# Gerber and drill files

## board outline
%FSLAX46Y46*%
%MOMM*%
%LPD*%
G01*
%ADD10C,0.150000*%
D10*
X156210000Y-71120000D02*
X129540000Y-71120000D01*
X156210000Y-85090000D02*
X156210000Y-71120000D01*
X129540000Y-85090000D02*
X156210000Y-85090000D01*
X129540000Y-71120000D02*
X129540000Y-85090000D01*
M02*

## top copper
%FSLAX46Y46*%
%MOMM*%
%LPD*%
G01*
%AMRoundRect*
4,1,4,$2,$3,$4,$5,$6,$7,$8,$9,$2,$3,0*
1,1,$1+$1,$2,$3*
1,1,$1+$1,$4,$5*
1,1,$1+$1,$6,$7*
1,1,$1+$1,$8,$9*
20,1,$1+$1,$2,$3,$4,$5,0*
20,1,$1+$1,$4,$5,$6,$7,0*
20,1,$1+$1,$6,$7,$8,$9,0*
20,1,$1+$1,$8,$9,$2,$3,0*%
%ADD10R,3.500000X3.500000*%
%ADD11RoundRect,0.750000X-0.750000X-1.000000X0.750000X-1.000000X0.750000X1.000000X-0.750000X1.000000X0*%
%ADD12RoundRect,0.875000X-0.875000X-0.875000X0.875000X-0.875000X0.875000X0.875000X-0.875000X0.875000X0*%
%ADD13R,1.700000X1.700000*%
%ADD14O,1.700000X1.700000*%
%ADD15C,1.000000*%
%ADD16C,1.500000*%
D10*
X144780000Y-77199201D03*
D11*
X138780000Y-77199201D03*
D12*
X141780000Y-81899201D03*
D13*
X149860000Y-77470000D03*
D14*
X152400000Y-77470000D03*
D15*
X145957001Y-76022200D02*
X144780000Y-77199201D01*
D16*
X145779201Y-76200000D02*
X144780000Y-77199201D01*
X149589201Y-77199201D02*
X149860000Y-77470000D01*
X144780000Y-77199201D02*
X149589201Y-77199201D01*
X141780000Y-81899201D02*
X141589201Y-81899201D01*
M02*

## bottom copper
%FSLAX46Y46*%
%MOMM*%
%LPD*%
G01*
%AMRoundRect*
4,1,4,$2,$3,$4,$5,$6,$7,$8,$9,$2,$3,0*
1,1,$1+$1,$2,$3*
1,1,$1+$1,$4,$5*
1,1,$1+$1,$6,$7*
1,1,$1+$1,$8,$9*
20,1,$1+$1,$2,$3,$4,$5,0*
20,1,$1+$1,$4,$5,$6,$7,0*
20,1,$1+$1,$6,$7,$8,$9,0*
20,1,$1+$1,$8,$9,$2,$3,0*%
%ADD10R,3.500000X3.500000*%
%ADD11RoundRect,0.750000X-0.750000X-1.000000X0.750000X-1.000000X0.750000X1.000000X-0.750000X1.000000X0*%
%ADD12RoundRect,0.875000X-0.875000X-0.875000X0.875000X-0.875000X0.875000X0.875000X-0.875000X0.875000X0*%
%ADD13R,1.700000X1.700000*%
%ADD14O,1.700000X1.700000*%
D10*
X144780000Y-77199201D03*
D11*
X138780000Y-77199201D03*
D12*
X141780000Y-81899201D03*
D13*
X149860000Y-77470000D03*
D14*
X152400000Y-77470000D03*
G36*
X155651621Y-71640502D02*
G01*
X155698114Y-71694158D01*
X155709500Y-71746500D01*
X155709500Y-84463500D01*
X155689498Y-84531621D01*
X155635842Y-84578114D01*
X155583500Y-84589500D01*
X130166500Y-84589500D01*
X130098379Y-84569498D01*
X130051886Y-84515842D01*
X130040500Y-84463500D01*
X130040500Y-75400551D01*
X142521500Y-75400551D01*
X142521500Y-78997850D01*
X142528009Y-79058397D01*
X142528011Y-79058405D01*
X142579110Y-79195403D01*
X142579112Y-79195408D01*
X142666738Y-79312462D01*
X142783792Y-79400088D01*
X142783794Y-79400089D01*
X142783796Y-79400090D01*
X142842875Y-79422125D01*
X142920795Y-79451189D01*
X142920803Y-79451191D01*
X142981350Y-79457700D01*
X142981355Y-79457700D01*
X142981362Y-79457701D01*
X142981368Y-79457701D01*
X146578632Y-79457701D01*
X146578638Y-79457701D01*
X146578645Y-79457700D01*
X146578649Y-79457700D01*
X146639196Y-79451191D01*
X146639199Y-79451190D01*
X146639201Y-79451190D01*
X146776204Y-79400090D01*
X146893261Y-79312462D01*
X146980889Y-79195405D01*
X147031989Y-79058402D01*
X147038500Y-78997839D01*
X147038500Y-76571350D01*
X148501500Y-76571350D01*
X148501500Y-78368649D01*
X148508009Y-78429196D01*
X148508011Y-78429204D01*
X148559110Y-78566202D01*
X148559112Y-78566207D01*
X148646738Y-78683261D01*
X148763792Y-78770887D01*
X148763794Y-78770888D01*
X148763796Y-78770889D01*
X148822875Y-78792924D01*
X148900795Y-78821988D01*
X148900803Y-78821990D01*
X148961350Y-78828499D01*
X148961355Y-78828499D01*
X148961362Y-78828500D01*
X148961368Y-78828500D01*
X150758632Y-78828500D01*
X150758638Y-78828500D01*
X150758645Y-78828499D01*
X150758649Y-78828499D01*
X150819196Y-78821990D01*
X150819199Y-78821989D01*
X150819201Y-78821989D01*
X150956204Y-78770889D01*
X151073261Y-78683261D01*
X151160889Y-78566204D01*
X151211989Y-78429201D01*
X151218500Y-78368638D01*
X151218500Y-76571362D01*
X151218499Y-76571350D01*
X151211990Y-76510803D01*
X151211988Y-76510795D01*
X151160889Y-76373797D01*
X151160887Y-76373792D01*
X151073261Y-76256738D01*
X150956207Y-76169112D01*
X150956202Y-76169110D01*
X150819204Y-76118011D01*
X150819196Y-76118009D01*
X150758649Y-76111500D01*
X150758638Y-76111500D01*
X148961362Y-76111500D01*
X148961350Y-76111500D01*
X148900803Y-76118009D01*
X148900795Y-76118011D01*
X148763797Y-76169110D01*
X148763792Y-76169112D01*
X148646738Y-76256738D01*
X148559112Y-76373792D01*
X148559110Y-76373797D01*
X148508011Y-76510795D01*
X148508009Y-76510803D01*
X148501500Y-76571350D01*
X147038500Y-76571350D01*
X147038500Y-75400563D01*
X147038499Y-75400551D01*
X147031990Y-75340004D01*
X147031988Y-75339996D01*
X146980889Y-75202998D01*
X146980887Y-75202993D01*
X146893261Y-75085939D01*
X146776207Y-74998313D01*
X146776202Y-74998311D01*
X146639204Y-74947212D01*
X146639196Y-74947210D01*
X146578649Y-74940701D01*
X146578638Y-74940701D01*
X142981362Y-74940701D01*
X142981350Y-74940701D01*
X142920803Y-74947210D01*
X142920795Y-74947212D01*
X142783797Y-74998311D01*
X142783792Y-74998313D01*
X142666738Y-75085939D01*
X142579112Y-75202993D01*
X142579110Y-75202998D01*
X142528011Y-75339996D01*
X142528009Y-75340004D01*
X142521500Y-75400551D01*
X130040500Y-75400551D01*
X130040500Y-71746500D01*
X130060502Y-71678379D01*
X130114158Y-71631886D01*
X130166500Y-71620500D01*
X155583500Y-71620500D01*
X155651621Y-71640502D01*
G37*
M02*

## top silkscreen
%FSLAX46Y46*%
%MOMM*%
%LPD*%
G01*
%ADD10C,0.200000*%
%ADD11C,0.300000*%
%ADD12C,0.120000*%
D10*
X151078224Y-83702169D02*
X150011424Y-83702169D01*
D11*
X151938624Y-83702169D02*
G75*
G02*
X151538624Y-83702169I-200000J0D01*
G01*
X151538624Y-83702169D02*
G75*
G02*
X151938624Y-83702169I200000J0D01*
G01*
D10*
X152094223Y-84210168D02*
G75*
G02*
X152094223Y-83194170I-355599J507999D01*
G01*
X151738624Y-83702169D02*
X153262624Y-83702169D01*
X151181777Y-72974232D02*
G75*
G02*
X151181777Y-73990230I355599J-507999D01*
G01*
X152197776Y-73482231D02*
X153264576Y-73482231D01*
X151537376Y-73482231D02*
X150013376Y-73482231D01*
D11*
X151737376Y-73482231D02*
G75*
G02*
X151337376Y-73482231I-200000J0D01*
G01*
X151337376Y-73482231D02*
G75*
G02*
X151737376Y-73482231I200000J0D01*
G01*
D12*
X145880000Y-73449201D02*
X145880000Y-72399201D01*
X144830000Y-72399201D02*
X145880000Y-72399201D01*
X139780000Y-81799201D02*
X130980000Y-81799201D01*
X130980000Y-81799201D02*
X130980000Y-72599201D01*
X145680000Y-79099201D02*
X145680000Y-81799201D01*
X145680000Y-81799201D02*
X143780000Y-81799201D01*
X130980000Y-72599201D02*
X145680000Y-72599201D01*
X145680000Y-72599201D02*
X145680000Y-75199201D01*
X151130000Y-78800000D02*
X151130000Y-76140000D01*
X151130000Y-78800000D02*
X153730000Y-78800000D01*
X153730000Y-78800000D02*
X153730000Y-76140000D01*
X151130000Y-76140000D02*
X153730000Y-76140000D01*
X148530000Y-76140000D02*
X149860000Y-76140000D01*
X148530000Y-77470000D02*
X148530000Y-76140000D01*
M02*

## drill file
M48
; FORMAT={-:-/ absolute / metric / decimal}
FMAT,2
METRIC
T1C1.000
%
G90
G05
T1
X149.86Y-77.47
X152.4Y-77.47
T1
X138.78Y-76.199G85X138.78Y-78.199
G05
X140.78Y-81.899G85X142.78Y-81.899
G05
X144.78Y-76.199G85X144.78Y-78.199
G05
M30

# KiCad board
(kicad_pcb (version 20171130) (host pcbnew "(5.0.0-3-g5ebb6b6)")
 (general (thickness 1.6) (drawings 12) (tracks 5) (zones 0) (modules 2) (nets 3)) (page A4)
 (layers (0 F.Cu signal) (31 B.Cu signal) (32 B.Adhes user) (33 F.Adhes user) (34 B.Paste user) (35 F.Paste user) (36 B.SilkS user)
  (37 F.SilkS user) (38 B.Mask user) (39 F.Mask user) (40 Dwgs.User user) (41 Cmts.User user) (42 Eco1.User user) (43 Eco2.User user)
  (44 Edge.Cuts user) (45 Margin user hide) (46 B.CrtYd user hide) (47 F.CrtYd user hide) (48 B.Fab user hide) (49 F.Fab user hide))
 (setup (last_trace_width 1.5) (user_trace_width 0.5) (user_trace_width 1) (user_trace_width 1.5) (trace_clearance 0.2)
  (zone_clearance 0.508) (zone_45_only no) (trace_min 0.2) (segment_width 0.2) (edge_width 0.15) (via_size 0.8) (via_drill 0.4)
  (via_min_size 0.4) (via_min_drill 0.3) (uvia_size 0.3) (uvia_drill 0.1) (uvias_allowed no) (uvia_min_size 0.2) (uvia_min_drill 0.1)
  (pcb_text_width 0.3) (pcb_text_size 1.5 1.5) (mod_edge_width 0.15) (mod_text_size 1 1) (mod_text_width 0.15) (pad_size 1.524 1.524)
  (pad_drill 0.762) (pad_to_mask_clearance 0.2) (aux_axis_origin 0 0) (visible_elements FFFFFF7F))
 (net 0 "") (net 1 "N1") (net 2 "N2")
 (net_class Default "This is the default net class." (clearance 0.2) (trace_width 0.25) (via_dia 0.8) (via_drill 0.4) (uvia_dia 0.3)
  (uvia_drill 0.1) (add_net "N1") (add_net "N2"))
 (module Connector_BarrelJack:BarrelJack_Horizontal (layer F.Cu) (at 144.78 77.199201)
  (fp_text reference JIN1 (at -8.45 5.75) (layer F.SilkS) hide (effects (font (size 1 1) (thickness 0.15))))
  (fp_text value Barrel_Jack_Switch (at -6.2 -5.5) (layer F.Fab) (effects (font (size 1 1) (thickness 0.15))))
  (fp_line (start 1.1 -3.75) (end 1.1 -4.8) (layer F.SilkS) (width 0.12))
  (fp_line (start 0.05 -4.8) (end 1.1 -4.8) (layer F.SilkS) (width 0.12))
  (fp_line (start -5 4.6) (end -13.8 4.6) (layer F.SilkS) (width 0.12))
  (fp_line (start -13.8 4.6) (end -13.8 -4.6) (layer F.SilkS) (width 0.12))
  (fp_line (start 0.9 1.9) (end 0.9 4.6) (layer F.SilkS) (width 0.12))
  (fp_line (start 0.9 4.6) (end -1 4.6) (layer F.SilkS) (width 0.12))
  (fp_line (start -13.8 -4.6) (end 0.9 -4.6) (layer F.SilkS) (width 0.12))
  (fp_line (start 0.9 -4.6) (end 0.9 -2) (layer F.SilkS) (width 0.12))
  (pad 1 thru_hole rect (at 0 0) (size 3.5 3.5) (drill oval 1 3) (layers *.Cu *.Mask) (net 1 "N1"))
  (pad 2 thru_hole roundrect (at -6 0) (size 3 3.5) (drill oval 1 3) (layers *.Cu *.Mask) (roundrect_rratio 0.25) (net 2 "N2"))
  (pad 3 thru_hole roundrect (at -3 4.7) (size 3.5 3.5) (drill oval 3 1) (layers *.Cu *.Mask) (roundrect_rratio 0.25) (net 2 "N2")))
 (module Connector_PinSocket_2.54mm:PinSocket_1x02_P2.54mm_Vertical (layer F.Cu) (at 149.86 77.47 90)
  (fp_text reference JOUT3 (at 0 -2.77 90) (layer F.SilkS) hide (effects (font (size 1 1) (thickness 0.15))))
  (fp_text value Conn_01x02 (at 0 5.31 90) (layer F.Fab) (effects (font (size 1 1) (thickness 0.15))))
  (fp_line (start -1.33 1.27) (end 1.33 1.27) (layer F.SilkS) (width 0.12))
  (fp_line (start -1.33 1.27) (end -1.33 3.87) (layer F.SilkS) (width 0.12))
  (fp_line (start -1.33 3.87) (end 1.33 3.87) (layer F.SilkS) (width 0.12))
  (fp_line (start 1.33 1.27) (end 1.33 3.87) (layer F.SilkS) (width 0.12))
  (fp_line (start 1.33 -1.33) (end 1.33 0) (layer F.SilkS) (width 0.12))
  (fp_line (start 0 -1.33) (end 1.33 -1.33) (layer F.SilkS) (width 0.12))
  (pad 1 thru_hole rect (at 0 0 90) (size 1.7 1.7) (drill 1) (layers *.Cu *.Mask) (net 1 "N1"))
  (pad 2 thru_hole oval (at 0 2.54 90) (size 1.7 1.7) (drill 1) (layers *.Cu *.Mask) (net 2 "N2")))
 (gr_line (start 156.21 71.12) (end 129.54 71.12) (layer Edge.Cuts) (width 0.15))
 (gr_line (start 156.21 85.09) (end 156.21 71.12) (layer Edge.Cuts) (width 0.15))
 (gr_line (start 129.54 85.09) (end 156.21 85.09) (layer Edge.Cuts) (width 0.15))
 (gr_line (start 129.54 71.12) (end 129.54 85.09) (layer Edge.Cuts) (width 0.15))
 (gr_line (start 151.078224 83.702169) (end 150.011424 83.702169) (layer F.SilkS) (width 0.2))
 (gr_circle (center 151.738624 83.702169) (end 151.938624 83.702169) (layer F.SilkS) (width 0.3))
 (gr_arc (start 151.738624 83.702169) (end 152.094223 83.19417) (angle -249.9840404) (layer F.SilkS) (width 0.2))
 (gr_line (start 151.738624 83.702169) (end 153.262624 83.702169) (layer F.SilkS) (width 0.2))
 (gr_arc (start 151.537376 73.482231) (end 151.181777 73.99023) (angle -249.9840404) (layer F.SilkS) (width 0.2))
 (gr_line (start 152.197776 73.482231) (end 153.264576 73.482231) (layer F.SilkS) (width 0.2))
 (gr_line (start 151.537376 73.482231) (end 150.013376 73.482231) (layer F.SilkS) (width 0.2))
 (gr_circle (center 151.537376 73.482231) (end 151.337376 73.482231) (layer F.SilkS) (width 0.3))
 (segment (start 145.957001 76.0222) (end 144.78 77.199201) (width 1) (layer F.Cu) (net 1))
 (segment (start 145.779201 76.2) (end 144.78 77.199201) (width 1.5) (layer F.Cu) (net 1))
 (segment (start 149.589201 77.199201) (end 149.86 77.47) (width 1.5) (layer F.Cu) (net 1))
 (segment (start 144.78 77.199201) (end 149.589201 77.199201) (width 1.5) (layer F.Cu) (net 1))
 (segment (start 141.78 81.899201) (end 141.589201 81.899201) (width 1.5) (layer F.Cu) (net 2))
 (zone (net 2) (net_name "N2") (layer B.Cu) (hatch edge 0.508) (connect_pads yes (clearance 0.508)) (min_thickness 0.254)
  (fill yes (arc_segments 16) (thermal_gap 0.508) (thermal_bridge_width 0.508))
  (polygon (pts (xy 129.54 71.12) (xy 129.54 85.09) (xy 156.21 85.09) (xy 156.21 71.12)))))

